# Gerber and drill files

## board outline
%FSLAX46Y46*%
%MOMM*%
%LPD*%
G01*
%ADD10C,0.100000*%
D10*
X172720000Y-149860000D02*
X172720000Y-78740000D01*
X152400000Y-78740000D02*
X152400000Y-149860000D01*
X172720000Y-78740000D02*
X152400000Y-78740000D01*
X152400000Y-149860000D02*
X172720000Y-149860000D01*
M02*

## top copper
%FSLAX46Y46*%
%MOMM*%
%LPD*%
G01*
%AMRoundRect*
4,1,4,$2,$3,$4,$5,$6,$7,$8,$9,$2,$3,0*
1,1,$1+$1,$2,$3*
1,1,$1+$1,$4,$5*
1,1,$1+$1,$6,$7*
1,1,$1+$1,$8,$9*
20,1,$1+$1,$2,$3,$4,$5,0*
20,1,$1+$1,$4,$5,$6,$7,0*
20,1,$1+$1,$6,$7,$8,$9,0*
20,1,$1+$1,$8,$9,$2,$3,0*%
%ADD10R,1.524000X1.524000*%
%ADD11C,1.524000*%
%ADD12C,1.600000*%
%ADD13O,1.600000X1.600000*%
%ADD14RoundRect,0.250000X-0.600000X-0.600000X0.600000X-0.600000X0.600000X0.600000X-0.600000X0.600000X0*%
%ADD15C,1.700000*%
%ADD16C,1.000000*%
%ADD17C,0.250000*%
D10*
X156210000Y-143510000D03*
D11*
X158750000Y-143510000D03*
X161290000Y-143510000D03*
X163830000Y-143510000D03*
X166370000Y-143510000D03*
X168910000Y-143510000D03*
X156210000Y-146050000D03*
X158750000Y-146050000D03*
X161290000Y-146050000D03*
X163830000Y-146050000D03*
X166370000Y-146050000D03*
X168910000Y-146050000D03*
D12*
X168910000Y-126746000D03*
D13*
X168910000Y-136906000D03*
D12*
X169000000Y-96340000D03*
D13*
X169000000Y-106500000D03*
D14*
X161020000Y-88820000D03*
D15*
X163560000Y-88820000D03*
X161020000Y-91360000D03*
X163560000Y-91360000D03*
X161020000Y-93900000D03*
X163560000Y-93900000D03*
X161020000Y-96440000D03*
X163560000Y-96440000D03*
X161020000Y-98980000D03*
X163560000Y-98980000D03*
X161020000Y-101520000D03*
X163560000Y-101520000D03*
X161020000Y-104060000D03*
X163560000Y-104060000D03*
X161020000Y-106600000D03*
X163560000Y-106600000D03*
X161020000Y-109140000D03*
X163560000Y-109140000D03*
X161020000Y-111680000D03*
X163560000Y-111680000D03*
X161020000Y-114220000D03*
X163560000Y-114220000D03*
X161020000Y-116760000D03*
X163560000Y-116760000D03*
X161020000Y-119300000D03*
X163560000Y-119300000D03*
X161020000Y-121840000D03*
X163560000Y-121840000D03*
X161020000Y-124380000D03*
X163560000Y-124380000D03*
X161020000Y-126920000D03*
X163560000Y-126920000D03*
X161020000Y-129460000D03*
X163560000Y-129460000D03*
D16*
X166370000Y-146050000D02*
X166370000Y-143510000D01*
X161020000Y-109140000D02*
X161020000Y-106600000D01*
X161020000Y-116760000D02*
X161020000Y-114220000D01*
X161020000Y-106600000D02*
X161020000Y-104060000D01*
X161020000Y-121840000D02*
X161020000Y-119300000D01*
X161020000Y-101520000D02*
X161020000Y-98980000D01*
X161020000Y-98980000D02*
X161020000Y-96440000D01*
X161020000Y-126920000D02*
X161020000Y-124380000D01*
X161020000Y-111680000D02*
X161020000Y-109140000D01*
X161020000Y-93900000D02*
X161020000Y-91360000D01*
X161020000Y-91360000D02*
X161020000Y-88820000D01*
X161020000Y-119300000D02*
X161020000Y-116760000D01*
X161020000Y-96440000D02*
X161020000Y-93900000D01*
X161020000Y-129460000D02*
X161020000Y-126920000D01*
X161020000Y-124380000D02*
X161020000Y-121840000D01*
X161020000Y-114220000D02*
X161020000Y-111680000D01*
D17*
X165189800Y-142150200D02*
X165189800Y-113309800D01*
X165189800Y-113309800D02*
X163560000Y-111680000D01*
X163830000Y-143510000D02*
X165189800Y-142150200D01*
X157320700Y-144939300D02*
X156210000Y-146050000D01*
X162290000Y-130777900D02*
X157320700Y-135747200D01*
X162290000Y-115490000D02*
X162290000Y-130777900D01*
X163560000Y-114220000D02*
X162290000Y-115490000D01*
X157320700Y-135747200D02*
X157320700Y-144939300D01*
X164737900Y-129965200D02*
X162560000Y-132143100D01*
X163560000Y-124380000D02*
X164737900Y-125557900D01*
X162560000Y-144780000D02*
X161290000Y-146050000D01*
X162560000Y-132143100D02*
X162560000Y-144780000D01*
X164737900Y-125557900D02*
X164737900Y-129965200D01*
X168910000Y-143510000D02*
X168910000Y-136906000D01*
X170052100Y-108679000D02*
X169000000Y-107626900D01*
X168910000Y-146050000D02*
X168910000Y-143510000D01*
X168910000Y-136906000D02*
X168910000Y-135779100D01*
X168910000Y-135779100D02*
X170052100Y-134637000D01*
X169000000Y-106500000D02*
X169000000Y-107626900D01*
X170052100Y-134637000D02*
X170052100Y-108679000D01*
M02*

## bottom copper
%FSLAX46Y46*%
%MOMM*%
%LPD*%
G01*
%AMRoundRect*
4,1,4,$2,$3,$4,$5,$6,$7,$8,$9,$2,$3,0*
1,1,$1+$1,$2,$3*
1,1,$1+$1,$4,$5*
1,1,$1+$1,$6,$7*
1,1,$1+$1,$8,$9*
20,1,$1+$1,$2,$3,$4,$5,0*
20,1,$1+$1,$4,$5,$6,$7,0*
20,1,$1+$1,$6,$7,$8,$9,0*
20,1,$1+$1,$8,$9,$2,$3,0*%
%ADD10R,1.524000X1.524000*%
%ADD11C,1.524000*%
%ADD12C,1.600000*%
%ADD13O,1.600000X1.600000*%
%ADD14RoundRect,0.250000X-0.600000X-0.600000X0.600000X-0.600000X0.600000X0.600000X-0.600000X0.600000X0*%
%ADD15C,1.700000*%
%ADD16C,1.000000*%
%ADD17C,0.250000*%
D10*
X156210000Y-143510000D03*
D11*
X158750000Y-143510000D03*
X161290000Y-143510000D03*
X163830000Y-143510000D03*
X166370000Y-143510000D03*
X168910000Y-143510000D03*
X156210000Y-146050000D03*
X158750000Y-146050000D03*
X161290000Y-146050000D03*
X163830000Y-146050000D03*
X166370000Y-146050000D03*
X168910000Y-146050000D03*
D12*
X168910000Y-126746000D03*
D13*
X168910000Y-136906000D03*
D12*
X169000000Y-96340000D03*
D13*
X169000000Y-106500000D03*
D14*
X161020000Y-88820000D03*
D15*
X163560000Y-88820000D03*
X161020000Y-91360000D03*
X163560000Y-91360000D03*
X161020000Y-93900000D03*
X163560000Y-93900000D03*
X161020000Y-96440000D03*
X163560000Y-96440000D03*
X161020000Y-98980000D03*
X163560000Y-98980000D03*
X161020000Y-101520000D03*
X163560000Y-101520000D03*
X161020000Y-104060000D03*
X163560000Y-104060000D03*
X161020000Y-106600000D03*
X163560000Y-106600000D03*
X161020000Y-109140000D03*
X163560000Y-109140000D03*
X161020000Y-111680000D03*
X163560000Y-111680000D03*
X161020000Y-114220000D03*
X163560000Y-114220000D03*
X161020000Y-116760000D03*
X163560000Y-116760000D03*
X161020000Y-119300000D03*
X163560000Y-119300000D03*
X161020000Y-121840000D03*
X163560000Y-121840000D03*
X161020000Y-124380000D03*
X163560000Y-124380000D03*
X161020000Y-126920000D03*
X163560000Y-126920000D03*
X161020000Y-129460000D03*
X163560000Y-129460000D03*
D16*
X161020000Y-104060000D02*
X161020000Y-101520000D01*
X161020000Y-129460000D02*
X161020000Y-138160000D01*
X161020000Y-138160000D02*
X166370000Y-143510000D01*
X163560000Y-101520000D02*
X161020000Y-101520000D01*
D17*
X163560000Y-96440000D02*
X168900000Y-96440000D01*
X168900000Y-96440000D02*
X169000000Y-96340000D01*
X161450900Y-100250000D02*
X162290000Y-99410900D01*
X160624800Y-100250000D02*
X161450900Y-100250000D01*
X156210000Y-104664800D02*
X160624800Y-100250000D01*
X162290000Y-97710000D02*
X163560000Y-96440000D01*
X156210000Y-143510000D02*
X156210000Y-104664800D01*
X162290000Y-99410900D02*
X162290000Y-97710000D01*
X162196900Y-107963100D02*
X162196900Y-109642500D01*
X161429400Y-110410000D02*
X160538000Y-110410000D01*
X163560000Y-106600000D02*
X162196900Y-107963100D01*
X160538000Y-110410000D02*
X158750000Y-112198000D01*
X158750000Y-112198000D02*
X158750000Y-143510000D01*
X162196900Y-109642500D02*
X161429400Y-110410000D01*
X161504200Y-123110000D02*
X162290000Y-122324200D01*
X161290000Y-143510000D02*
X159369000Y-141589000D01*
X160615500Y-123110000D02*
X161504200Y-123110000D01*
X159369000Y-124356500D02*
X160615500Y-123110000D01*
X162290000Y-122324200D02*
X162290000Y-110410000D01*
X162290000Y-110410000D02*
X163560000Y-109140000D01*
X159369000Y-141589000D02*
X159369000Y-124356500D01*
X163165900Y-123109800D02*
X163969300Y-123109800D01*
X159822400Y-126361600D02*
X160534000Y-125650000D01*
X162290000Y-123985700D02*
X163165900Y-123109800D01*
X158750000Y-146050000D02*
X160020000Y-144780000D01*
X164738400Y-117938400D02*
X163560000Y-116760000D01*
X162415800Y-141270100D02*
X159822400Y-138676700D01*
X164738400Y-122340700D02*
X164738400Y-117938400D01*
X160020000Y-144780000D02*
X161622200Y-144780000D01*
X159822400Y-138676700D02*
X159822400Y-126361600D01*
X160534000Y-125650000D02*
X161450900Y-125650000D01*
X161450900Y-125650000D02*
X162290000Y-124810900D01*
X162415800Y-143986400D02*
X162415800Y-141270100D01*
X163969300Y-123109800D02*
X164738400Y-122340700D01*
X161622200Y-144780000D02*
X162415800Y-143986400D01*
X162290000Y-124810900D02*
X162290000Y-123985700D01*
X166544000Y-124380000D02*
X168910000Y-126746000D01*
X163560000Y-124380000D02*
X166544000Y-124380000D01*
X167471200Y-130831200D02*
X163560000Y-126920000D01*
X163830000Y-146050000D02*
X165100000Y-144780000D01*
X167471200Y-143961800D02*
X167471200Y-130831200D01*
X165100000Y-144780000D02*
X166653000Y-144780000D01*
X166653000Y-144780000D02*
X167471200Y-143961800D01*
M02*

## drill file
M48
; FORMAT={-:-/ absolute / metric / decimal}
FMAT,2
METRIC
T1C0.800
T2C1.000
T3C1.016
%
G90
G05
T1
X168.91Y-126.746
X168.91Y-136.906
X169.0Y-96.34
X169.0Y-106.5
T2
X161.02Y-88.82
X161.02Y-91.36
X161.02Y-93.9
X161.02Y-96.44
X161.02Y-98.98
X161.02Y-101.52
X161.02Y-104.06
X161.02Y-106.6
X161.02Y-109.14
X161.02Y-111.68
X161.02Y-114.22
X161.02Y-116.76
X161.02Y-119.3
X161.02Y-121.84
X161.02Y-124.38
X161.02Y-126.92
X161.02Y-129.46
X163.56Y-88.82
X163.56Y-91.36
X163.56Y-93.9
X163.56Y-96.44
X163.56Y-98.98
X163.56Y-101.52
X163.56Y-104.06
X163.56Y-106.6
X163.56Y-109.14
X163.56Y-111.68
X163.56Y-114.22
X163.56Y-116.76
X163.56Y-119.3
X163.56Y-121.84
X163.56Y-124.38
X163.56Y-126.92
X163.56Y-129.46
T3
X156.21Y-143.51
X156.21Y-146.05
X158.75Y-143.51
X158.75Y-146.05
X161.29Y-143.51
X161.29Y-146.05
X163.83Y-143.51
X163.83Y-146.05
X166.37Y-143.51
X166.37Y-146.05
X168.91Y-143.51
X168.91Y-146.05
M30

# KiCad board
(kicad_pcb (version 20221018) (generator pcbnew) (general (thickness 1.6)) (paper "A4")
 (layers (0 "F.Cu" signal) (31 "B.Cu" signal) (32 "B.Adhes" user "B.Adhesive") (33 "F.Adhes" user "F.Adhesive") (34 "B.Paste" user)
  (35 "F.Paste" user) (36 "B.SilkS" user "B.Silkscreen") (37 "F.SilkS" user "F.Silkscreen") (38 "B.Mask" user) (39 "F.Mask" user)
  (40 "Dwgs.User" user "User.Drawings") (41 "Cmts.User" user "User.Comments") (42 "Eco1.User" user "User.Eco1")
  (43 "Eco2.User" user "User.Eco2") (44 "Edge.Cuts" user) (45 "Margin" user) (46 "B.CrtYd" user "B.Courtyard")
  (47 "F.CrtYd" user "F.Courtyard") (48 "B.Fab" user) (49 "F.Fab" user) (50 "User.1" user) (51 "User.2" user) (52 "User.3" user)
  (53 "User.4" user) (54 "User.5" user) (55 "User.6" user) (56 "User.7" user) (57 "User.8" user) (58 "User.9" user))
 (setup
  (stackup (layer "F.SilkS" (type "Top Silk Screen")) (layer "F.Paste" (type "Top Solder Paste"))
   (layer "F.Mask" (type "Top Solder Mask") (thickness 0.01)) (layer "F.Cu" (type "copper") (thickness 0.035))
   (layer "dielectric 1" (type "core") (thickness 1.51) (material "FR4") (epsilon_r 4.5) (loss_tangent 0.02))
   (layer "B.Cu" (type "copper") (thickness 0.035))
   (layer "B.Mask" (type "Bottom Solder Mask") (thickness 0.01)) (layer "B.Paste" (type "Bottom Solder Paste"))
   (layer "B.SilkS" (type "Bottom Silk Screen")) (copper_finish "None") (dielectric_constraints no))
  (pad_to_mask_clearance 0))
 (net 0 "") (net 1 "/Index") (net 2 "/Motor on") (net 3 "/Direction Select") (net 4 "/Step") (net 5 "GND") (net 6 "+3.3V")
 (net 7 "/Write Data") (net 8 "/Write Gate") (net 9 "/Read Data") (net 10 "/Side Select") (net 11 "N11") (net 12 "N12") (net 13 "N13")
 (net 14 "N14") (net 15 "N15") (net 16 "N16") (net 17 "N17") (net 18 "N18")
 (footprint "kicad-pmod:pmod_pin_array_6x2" (layer "F.Cu") (at 162.56 144.78 90)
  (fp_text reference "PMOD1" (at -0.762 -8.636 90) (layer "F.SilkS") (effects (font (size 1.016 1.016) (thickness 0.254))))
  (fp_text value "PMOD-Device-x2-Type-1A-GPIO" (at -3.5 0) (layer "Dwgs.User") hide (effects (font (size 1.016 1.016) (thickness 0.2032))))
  (pad "1" thru_hole rect (at 1.27 -6.35 90) (size 1.524 1.524) (drill 1.016) (layers "*.Cu" "*.Mask" "F.SilkS") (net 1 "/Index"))
  (pad "2" thru_hole circle (at 1.27 -3.81) (size 1.524 1.524) (drill 1.016) (layers "*.Cu" "*.Mask" "F.SilkS") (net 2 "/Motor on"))
  (pad "3" thru_hole circle (at 1.27 -1.27) (size 1.524 1.524) (drill 1.016) (layers "*.Cu" "*.Mask" "F.SilkS") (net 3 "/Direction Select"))
  (pad "4" thru_hole circle (at 1.27 1.27) (size 1.524 1.524) (drill 1.016) (layers "*.Cu" "*.Mask" "F.SilkS") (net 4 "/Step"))
  (pad "5" thru_hole circle (at 1.27 3.81) (size 1.524 1.524) (drill 1.016) (layers "*.Cu" "*.Mask" "F.SilkS") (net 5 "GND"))
  (pad "6" thru_hole circle (at 1.27 6.35) (size 1.524 1.524) (drill 1.016) (layers "*.Cu" "*.Mask" "F.SilkS") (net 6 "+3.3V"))
  (pad "7" thru_hole circle (at -1.27 -6.35) (size 1.524 1.524) (drill 1.016) (layers "*.Cu" "*.Mask" "F.SilkS") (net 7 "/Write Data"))
  (pad "8" thru_hole circle (at -1.27 -3.81) (size 1.524 1.524) (drill 1.016) (layers "*.Cu" "*.Mask" "F.SilkS") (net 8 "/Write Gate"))
  (pad "9" thru_hole circle (at -1.27 -1.27) (size 1.524 1.524) (drill 1.016) (layers "*.Cu" "*.Mask" "F.SilkS") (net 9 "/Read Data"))
  (pad "10" thru_hole circle (at -1.27 1.27) (size 1.524 1.524) (drill 1.016) (layers "*.Cu" "*.Mask" "F.SilkS") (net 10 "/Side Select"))
  (pad "11" thru_hole circle (at -1.27 3.81) (size 1.524 1.524) (drill 1.016) (layers "*.Cu" "*.Mask" "F.SilkS") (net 5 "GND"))
  (pad "12" thru_hole circle (at -1.27 6.35) (size 1.524 1.524) (drill 1.016) (layers "*.Cu" "*.Mask" "F.SilkS") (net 6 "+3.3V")))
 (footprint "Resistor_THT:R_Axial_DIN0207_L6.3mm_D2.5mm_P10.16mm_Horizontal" (layer "F.Cu") (at 168.91 126.746 -90)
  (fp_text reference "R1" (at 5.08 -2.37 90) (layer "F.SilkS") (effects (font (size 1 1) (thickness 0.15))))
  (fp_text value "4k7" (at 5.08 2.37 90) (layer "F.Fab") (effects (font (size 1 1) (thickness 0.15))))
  (pad "1" thru_hole circle (at 0 0 270) (size 1.6 1.6) (drill 0.8) (layers "*.Cu" "*.Mask") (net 9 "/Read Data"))
  (pad "2" thru_hole oval (at 10.16 0 270) (size 1.6 1.6) (drill 0.8) (layers "*.Cu" "*.Mask") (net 6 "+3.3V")))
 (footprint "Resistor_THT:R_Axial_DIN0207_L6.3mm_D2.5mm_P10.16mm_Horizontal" (layer "F.Cu") (at 169 96.34 -90)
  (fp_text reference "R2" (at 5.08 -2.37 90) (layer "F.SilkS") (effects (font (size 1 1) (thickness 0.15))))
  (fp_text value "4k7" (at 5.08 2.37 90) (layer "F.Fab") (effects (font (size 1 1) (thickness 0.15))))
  (pad "1" thru_hole circle (at 0 0 270) (size 1.6 1.6) (drill 0.8) (layers "*.Cu" "*.Mask") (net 1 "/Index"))
  (pad "2" thru_hole oval (at 10.16 0 270) (size 1.6 1.6) (drill 0.8) (layers "*.Cu" "*.Mask") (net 6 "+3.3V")))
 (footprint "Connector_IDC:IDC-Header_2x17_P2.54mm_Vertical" (layer "F.Cu") (at 161.02 88.82)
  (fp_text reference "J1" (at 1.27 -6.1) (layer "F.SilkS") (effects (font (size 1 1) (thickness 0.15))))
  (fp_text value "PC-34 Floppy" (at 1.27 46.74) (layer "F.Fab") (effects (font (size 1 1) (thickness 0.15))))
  (pad "1" thru_hole roundrect (at 0 0) (size 1.7 1.7) (drill 1) (layers "*.Cu" "*.Mask") (roundrect_rratio 0.1470588235) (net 5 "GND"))
  (pad "2" thru_hole circle (at 2.54 0) (size 1.7 1.7) (drill 1) (layers "*.Cu" "*.Mask") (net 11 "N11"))
  (pad "3" thru_hole circle (at 0 2.54) (size 1.7 1.7) (drill 1) (layers "*.Cu" "*.Mask") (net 5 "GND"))
  (pad "4" thru_hole circle (at 2.54 2.54) (size 1.7 1.7) (drill 1) (layers "*.Cu" "*.Mask") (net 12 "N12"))
  (pad "5" thru_hole circle (at 0 5.08) (size 1.7 1.7) (drill 1) (layers "*.Cu" "*.Mask") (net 5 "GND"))
  (pad "6" thru_hole circle (at 2.54 5.08) (size 1.7 1.7) (drill 1) (layers "*.Cu" "*.Mask") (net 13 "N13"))
  (pad "7" thru_hole circle (at 0 7.62) (size 1.7 1.7) (drill 1) (layers "*.Cu" "*.Mask") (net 5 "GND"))
  (pad "8" thru_hole circle (at 2.54 7.62) (size 1.7 1.7) (drill 1) (layers "*.Cu" "*.Mask") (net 1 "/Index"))
  (pad "9" thru_hole circle (at 0 10.16) (size 1.7 1.7) (drill 1) (layers "*.Cu" "*.Mask") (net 5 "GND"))
  (pad "10" thru_hole circle (at 2.54 10.16) (size 1.7 1.7) (drill 1) (layers "*.Cu" "*.Mask") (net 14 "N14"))
  (pad "11" thru_hole circle (at 0 12.7) (size 1.7 1.7) (drill 1) (layers "*.Cu" "*.Mask") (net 5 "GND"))
  (pad "12" thru_hole circle (at 2.54 12.7) (size 1.7 1.7) (drill 1) (layers "*.Cu" "*.Mask") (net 5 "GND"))
  (pad "13" thru_hole circle (at 0 15.24) (size 1.7 1.7) (drill 1) (layers "*.Cu" "*.Mask") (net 5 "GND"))
  (pad "14" thru_hole circle (at 2.54 15.24) (size 1.7 1.7) (drill 1) (layers "*.Cu" "*.Mask") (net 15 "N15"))
  (pad "15" thru_hole circle (at 0 17.78) (size 1.7 1.7) (drill 1) (layers "*.Cu" "*.Mask") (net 5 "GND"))
  (pad "16" thru_hole circle (at 2.54 17.78) (size 1.7 1.7) (drill 1) (layers "*.Cu" "*.Mask") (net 2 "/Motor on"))
  (pad "17" thru_hole circle (at 0 20.32) (size 1.7 1.7) (drill 1) (layers "*.Cu" "*.Mask") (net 5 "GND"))
  (pad "18" thru_hole circle (at 2.54 20.32) (size 1.7 1.7) (drill 1) (layers "*.Cu" "*.Mask") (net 3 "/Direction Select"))
  (pad "19" thru_hole circle (at 0 22.86) (size 1.7 1.7) (drill 1) (layers "*.Cu" "*.Mask") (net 5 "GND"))
  (pad "20" thru_hole circle (at 2.54 22.86) (size 1.7 1.7) (drill 1) (layers "*.Cu" "*.Mask") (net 4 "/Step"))
  (pad "21" thru_hole circle (at 0 25.4) (size 1.7 1.7) (drill 1) (layers "*.Cu" "*.Mask") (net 5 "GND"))
  (pad "22" thru_hole circle (at 2.54 25.4) (size 1.7 1.7) (drill 1) (layers "*.Cu" "*.Mask") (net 7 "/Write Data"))
  (pad "23" thru_hole circle (at 0 27.94) (size 1.7 1.7) (drill 1) (layers "*.Cu" "*.Mask") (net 5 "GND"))
  (pad "24" thru_hole circle (at 2.54 27.94) (size 1.7 1.7) (drill 1) (layers "*.Cu" "*.Mask") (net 8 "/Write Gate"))
  (pad "25" thru_hole circle (at 0 30.48) (size 1.7 1.7) (drill 1) (layers "*.Cu" "*.Mask") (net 5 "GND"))
  (pad "26" thru_hole circle (at 2.54 30.48) (size 1.7 1.7) (drill 1) (layers "*.Cu" "*.Mask") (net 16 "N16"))
  (pad "27" thru_hole circle (at 0 33.02) (size 1.7 1.7) (drill 1) (layers "*.Cu" "*.Mask") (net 5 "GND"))
  (pad "28" thru_hole circle (at 2.54 33.02) (size 1.7 1.7) (drill 1) (layers "*.Cu" "*.Mask") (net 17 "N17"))
  (pad "29" thru_hole circle (at 0 35.56) (size 1.7 1.7) (drill 1) (layers "*.Cu" "*.Mask") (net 5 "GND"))
  (pad "30" thru_hole circle (at 2.54 35.56) (size 1.7 1.7) (drill 1) (layers "*.Cu" "*.Mask") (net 9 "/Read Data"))
  (pad "31" thru_hole circle (at 0 38.1) (size 1.7 1.7) (drill 1) (layers "*.Cu" "*.Mask") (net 5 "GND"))
  (pad "32" thru_hole circle (at 2.54 38.1) (size 1.7 1.7) (drill 1) (layers "*.Cu" "*.Mask") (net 10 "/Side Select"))
  (pad "33" thru_hole circle (at 0 40.64) (size 1.7 1.7) (drill 1) (layers "*.Cu" "*.Mask") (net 5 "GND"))
  (pad "34" thru_hole circle (at 2.54 40.64) (size 1.7 1.7) (drill 1) (layers "*.Cu" "*.Mask") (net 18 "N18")))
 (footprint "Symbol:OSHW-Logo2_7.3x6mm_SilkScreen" (layer "F.Cu") (at 161.5 138.75)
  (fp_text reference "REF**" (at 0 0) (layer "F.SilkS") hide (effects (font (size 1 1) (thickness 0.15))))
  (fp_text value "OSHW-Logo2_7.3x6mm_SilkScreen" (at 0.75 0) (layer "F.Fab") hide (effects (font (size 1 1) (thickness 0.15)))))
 (gr_line (start 172.72 149.86) (end 172.72 78.74) (stroke (width 0.1) (type default)) (layer "Edge.Cuts"))
 (gr_line (start 152.4 78.74) (end 152.4 149.86) (stroke (width 0.1) (type default)) (layer "Edge.Cuts"))
 (gr_line (start 172.72 78.74) (end 152.4 78.74) (stroke (width 0.1) (type default)) (layer "Edge.Cuts"))
 (gr_line (start 152.4 149.86) (end 172.72 149.86) (stroke (width 0.1) (type default)) (layer "Edge.Cuts"))
 (segment (start 166.37 146.05) (end 166.37 143.51) (width 1) (layer "F.Cu") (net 5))
 (segment (start 161.02 109.14) (end 161.02 106.6) (width 1) (layer "F.Cu") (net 5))
 (segment (start 161.02 116.76) (end 161.02 114.22) (width 1) (layer "F.Cu") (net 5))
 (segment (start 161.02 106.6) (end 161.02 104.06) (width 1) (layer "F.Cu") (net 5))
 (segment (start 161.02 121.84) (end 161.02 119.3) (width 1) (layer "F.Cu") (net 5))
 (segment (start 161.02 101.52) (end 161.02 98.98) (width 1) (layer "F.Cu") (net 5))
 (segment (start 161.02 98.98) (end 161.02 96.44) (width 1) (layer "F.Cu") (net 5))
 (segment (start 161.02 126.92) (end 161.02 124.38) (width 1) (layer "F.Cu") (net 5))
 (segment (start 161.02 111.68) (end 161.02 109.14) (width 1) (layer "F.Cu") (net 5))
 (segment (start 161.02 93.9) (end 161.02 91.36) (width 1) (layer "F.Cu") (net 5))
 (segment (start 161.02 91.36) (end 161.02 88.82) (width 1) (layer "F.Cu") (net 5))
 (segment (start 161.02 119.3) (end 161.02 116.76) (width 1) (layer "F.Cu") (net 5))
 (segment (start 161.02 96.44) (end 161.02 93.9) (width 1) (layer "F.Cu") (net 5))
 (segment (start 161.02 129.46) (end 161.02 126.92) (width 1) (layer "F.Cu") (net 5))
 (segment (start 161.02 124.38) (end 161.02 121.84) (width 1) (layer "F.Cu") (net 5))
 (segment (start 161.02 114.22) (end 161.02 111.68) (width 1) (layer "F.Cu") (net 5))
 (segment (start 161.02 104.06) (end 161.02 101.52) (width 1) (layer "B.Cu") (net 5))
 (segment (start 161.02 129.46) (end 161.02 138.16) (width 1) (layer "B.Cu") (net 5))
 (segment (start 161.02 138.16) (end 166.37 143.51) (width 1) (layer "B.Cu") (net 5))
 (segment (start 163.56 101.52) (end 161.02 101.52) (width 1) (layer "B.Cu") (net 5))
 (segment (start 163.56 96.44) (end 168.9 96.44) (width 0.25) (layer "B.Cu") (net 1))
 (segment (start 168.9 96.44) (end 169 96.34) (width 0.25) (layer "B.Cu") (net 1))
 (segment (start 161.4509 100.25) (end 162.29 99.4109) (width 0.25) (layer "B.Cu") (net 1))
 (segment (start 160.6248 100.25) (end 161.4509 100.25) (width 0.25) (layer "B.Cu") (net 1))
 (segment (start 156.21 104.6648) (end 160.6248 100.25) (width 0.25) (layer "B.Cu") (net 1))
 (segment (start 162.29 97.71) (end 163.56 96.44) (width 0.25) (layer "B.Cu") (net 1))
 (segment (start 156.21 143.51) (end 156.21 104.6648) (width 0.25) (layer "B.Cu") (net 1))
 (segment (start 162.29 99.4109) (end 162.29 97.71) (width 0.25) (layer "B.Cu") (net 1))
 (segment (start 162.1969 107.9631) (end 162.1969 109.6425) (width 0.25) (layer "B.Cu") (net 2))
 (segment (start 161.4294 110.41) (end 160.538 110.41) (width 0.25) (layer "B.Cu") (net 2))
 (segment (start 163.56 106.6) (end 162.1969 107.9631) (width 0.25) (layer "B.Cu") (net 2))
 (segment (start 160.538 110.41) (end 158.75 112.198) (width 0.25) (layer "B.Cu") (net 2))
 (segment (start 158.75 112.198) (end 158.75 143.51) (width 0.25) (layer "B.Cu") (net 2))
 (segment (start 162.1969 109.6425) (end 161.4294 110.41) (width 0.25) (layer "B.Cu") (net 2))
 (segment (start 161.5042 123.11) (end 162.29 122.3242) (width 0.25) (layer "B.Cu") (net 3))
 (segment (start 161.29 143.51) (end 159.369 141.589) (width 0.25) (layer "B.Cu") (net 3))
 (segment (start 160.6155 123.11) (end 161.5042 123.11) (width 0.25) (layer "B.Cu") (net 3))
 (segment (start 159.369 124.3565) (end 160.6155 123.11) (width 0.25) (layer "B.Cu") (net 3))
 (segment (start 162.29 122.3242) (end 162.29 110.41) (width 0.25) (layer "B.Cu") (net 3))
 (segment (start 162.29 110.41) (end 163.56 109.14) (width 0.25) (layer "B.Cu") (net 3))
 (segment (start 159.369 141.589) (end 159.369 124.3565) (width 0.25) (layer "B.Cu") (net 3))
 (segment (start 165.1898 142.1502) (end 165.1898 113.3098) (width 0.25) (layer "F.Cu") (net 4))
 (segment (start 165.1898 113.3098) (end 163.56 111.68) (width 0.25) (layer "F.Cu") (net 4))
 (segment (start 163.83 143.51) (end 165.1898 142.1502) (width 0.25) (layer "F.Cu") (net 4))
 (segment (start 157.3207 144.9393) (end 156.21 146.05) (width 0.25) (layer "F.Cu") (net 7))
 (segment (start 162.29 130.7779) (end 157.3207 135.7472) (width 0.25) (layer "F.Cu") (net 7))
 (segment (start 162.29 115.49) (end 162.29 130.7779) (width 0.25) (layer "F.Cu") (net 7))
 (segment (start 163.56 114.22) (end 162.29 115.49) (width 0.25) (layer "F.Cu") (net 7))
 (segment (start 157.3207 135.7472) (end 157.3207 144.9393) (width 0.25) (layer "F.Cu") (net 7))
 (segment (start 163.1659 123.1098) (end 163.9693 123.1098) (width 0.25) (layer "B.Cu") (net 8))
 (segment (start 159.8224 126.3616) (end 160.534 125.65) (width 0.25) (layer "B.Cu") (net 8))
 (segment (start 162.29 123.9857) (end 163.1659 123.1098) (width 0.25) (layer "B.Cu") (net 8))
 (segment (start 158.75 146.05) (end 160.02 144.78) (width 0.25) (layer "B.Cu") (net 8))
 (segment (start 164.7384 117.9384) (end 163.56 116.76) (width 0.25) (layer "B.Cu") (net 8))
 (segment (start 162.4158 141.2701) (end 159.8224 138.6767) (width 0.25) (layer "B.Cu") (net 8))
 (segment (start 164.7384 122.3407) (end 164.7384 117.9384) (width 0.25) (layer "B.Cu") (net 8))
 (segment (start 160.02 144.78) (end 161.6222 144.78) (width 0.25) (layer "B.Cu") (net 8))
 (segment (start 159.8224 138.6767) (end 159.8224 126.3616) (width 0.25) (layer "B.Cu") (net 8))
 (segment (start 160.534 125.65) (end 161.4509 125.65) (width 0.25) (layer "B.Cu") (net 8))
 (segment (start 161.4509 125.65) (end 162.29 124.8109) (width 0.25) (layer "B.Cu") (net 8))
 (segment (start 162.4158 143.9864) (end 162.4158 141.2701) (width 0.25) (layer "B.Cu") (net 8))
 (segment (start 163.9693 123.1098) (end 164.7384 122.3407) (width 0.25) (layer "B.Cu") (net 8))
 (segment (start 161.6222 144.78) (end 162.4158 143.9864) (width 0.25) (layer "B.Cu") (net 8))
 (segment (start 162.29 124.8109) (end 162.29 123.9857) (width 0.25) (layer "B.Cu") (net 8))
 (segment (start 164.7379 129.9652) (end 162.56 132.1431) (width 0.25) (layer "F.Cu") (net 9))
 (segment (start 163.56 124.38) (end 164.7379 125.5579) (width 0.25) (layer "F.Cu") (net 9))
 (segment (start 162.56 144.78) (end 161.29 146.05) (width 0.25) (layer "F.Cu") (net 9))
 (segment (start 162.56 132.1431) (end 162.56 144.78) (width 0.25) (layer "F.Cu") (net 9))
 (segment (start 164.7379 125.5579) (end 164.7379 129.9652) (width 0.25) (layer "F.Cu") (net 9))
 (segment (start 166.544 124.38) (end 168.91 126.746) (width 0.25) (layer "B.Cu") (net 9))
 (segment (start 163.56 124.38) (end 166.544 124.38) (width 0.25) (layer "B.Cu") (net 9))
 (segment (start 167.4712 130.8312) (end 163.56 126.92) (width 0.25) (layer "B.Cu") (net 10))
 (segment (start 163.83 146.05) (end 165.1 144.78) (width 0.25) (layer "B.Cu") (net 10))
 (segment (start 167.4712 143.9618) (end 167.4712 130.8312) (width 0.25) (layer "B.Cu") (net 10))
 (segment (start 165.1 144.78) (end 166.653 144.78) (width 0.25) (layer "B.Cu") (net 10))
 (segment (start 166.653 144.78) (end 167.4712 143.9618) (width 0.25) (layer "B.Cu") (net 10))
 (segment (start 168.91 143.51) (end 168.91 136.906) (width 0.25) (layer "F.Cu") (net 6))
 (segment (start 170.0521 108.679) (end 169 107.6269) (width 0.25) (layer "F.Cu") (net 6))
 (segment (start 168.91 146.05) (end 168.91 143.51) (width 0.25) (layer "F.Cu") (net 6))
 (segment (start 168.91 136.906) (end 168.91 135.7791) (width 0.25) (layer "F.Cu") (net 6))
 (segment (start 168.91 135.7791) (end 170.0521 134.637) (width 0.25) (layer "F.Cu") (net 6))
 (segment (start 169 106.5) (end 169 107.6269) (width 0.25) (layer "F.Cu") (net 6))
 (segment (start 170.0521 134.637) (end 170.0521 108.679) (width 0.25) (layer "F.Cu") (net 6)))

